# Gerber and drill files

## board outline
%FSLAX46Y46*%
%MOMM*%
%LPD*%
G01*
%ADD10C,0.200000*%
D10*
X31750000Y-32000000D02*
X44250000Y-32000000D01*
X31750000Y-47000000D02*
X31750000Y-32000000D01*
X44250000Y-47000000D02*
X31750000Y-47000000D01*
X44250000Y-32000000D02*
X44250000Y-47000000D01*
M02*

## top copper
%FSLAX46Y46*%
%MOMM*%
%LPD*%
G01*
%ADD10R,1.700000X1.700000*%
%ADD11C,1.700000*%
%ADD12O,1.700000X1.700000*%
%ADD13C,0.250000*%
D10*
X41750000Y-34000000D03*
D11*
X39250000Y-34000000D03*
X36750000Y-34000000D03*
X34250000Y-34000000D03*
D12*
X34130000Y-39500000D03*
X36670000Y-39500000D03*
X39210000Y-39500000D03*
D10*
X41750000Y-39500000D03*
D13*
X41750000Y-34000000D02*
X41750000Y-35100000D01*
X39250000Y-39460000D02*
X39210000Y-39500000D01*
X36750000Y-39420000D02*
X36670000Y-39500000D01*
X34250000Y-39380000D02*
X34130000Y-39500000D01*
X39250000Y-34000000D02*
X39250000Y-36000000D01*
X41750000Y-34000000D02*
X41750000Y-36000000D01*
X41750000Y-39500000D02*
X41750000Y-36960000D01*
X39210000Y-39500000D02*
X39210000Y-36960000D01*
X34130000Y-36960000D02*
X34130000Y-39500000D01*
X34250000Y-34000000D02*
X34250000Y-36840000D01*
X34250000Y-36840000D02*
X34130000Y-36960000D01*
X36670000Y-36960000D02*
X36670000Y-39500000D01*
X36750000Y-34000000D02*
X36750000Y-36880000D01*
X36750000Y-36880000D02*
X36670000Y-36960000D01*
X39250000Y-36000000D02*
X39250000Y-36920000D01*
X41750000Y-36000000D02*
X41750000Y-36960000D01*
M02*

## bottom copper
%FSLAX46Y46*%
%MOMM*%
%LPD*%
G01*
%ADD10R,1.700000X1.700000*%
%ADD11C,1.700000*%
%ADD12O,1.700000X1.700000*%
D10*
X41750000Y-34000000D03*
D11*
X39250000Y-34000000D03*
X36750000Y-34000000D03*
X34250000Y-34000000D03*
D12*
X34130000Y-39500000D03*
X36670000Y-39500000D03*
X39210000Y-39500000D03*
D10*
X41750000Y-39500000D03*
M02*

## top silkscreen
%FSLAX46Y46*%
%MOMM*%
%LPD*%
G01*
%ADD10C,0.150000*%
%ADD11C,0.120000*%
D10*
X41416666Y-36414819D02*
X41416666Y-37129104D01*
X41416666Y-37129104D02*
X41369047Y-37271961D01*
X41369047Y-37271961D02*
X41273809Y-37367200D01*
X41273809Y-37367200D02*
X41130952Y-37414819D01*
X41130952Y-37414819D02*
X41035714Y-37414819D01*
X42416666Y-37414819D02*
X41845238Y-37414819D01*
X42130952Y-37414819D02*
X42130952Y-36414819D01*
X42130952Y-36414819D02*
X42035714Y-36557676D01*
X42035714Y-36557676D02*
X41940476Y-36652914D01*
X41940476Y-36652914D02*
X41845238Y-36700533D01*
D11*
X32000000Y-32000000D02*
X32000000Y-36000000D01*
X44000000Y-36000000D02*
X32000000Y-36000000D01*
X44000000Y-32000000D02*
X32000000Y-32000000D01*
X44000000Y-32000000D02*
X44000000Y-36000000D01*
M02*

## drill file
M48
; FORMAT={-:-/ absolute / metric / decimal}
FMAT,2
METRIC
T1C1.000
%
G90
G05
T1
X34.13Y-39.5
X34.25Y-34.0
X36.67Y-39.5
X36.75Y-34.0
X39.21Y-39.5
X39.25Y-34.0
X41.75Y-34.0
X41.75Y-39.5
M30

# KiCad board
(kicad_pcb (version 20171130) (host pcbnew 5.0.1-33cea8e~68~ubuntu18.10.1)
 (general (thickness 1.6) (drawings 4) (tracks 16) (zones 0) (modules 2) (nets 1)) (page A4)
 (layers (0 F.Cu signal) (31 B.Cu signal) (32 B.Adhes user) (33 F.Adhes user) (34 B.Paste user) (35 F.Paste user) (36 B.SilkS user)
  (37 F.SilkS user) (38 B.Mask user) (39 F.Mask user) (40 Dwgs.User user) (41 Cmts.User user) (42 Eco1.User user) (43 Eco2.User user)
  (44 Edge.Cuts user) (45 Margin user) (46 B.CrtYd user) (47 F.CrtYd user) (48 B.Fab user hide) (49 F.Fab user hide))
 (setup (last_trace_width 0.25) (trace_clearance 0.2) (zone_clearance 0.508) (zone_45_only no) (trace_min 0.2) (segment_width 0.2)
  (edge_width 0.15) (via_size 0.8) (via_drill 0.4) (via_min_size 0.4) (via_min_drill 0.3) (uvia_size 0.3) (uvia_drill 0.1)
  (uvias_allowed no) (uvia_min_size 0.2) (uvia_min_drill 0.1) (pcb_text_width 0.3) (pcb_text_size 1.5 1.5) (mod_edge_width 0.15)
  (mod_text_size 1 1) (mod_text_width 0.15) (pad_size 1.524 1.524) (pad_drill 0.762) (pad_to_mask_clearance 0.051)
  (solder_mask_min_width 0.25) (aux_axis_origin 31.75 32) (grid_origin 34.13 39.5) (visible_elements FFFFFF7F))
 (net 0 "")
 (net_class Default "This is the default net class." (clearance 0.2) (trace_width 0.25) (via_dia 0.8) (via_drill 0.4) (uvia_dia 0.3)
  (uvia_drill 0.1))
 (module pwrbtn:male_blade (layer F.Cu) (at 38 34 180)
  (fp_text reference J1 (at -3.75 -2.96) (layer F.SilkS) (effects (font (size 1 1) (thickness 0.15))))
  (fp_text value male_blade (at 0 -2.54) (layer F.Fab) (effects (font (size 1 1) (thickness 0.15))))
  (fp_line (start 6 2) (end 6 -2) (layer F.SilkS) (width 0.12))
  (fp_line (start -6 -2) (end 6 -2) (layer F.SilkS) (width 0.12))
  (fp_line (start -6 2) (end 6 2) (layer F.SilkS) (width 0.12))
  (fp_line (start -6 2) (end -6 -2) (layer F.SilkS) (width 0.12))
  (pad 1 thru_hole rect (at -3.75 0 270) (size 1.7 1.7) (drill 1) (layers *.Cu *.Mask))
  (pad 2 thru_hole circle (at -1.25 0 270) (size 1.7 1.7) (drill 1) (layers *.Cu *.Mask))
  (pad 3 thru_hole circle (at 1.25 0 270) (size 1.7 1.7) (drill 1) (layers *.Cu *.Mask))
  (pad 4 thru_hole circle (at 3.75 0 270) (size 1.7 1.7) (drill 1) (layers *.Cu *.Mask)))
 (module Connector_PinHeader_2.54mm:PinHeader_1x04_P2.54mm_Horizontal (layer B.Cu) (at 41.75 39.5 90)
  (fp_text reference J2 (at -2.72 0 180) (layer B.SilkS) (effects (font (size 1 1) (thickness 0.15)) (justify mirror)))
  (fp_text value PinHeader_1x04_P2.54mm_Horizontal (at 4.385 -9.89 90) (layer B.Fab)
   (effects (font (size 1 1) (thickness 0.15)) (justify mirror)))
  (pad 4 thru_hole oval (at 0 -7.62 90) (size 1.7 1.7) (drill 1) (layers *.Cu *.Mask))
  (pad 3 thru_hole oval (at 0 -5.08 90) (size 1.7 1.7) (drill 1) (layers *.Cu *.Mask))
  (pad 2 thru_hole oval (at 0 -2.54 90) (size 1.7 1.7) (drill 1) (layers *.Cu *.Mask))
  (pad 1 thru_hole rect (at 0 0 90) (size 1.7 1.7) (drill 1) (layers *.Cu *.Mask)))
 (gr_line (start 31.75 32) (end 44.25 32) (layer Edge.Cuts) (width 0.2))
 (gr_line (start 31.75 47) (end 31.75 32) (layer Edge.Cuts) (width 0.2))
 (gr_line (start 44.25 47) (end 31.75 47) (layer Edge.Cuts) (width 0.2))
 (gr_line (start 44.25 32) (end 44.25 47) (layer Edge.Cuts) (width 0.2))
 (segment (start 41.75 34) (end 41.75 35.1) (width 0.25) (layer F.Cu) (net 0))
 (segment (start 39.25 39.46) (end 39.21 39.5) (width 0.25) (layer F.Cu) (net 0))
 (segment (start 36.75 39.42) (end 36.67 39.5) (width 0.25) (layer F.Cu) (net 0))
 (segment (start 34.25 39.38) (end 34.13 39.5) (width 0.25) (layer F.Cu) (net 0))
 (segment (start 39.25 34) (end 39.25 36) (width 0.25) (layer F.Cu) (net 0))
 (segment (start 41.75 34) (end 41.75 36) (width 0.25) (layer F.Cu) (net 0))
 (segment (start 41.75 39.5) (end 41.75 36.96) (width 0.25) (layer F.Cu) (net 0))
 (segment (start 39.21 39.5) (end 39.21 36.96) (width 0.25) (layer F.Cu) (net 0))
 (segment (start 34.13 36.96) (end 34.13 39.5) (width 0.25) (layer F.Cu) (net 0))
 (segment (start 34.25 34) (end 34.25 36.84) (width 0.25) (layer F.Cu) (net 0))
 (segment (start 34.25 36.84) (end 34.13 36.96) (width 0.25) (layer F.Cu) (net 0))
 (segment (start 36.67 36.96) (end 36.67 39.5) (width 0.25) (layer F.Cu) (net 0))
 (segment (start 36.75 34) (end 36.75 36.88) (width 0.25) (layer F.Cu) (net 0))
 (segment (start 36.75 36.88) (end 36.67 36.96) (width 0.25) (layer F.Cu) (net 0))
 (segment (start 39.25 36) (end 39.25 36.92) (width 0.25) (layer F.Cu) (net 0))
 (segment (start 41.75 36) (end 41.75 36.96) (width 0.25) (layer F.Cu) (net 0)))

